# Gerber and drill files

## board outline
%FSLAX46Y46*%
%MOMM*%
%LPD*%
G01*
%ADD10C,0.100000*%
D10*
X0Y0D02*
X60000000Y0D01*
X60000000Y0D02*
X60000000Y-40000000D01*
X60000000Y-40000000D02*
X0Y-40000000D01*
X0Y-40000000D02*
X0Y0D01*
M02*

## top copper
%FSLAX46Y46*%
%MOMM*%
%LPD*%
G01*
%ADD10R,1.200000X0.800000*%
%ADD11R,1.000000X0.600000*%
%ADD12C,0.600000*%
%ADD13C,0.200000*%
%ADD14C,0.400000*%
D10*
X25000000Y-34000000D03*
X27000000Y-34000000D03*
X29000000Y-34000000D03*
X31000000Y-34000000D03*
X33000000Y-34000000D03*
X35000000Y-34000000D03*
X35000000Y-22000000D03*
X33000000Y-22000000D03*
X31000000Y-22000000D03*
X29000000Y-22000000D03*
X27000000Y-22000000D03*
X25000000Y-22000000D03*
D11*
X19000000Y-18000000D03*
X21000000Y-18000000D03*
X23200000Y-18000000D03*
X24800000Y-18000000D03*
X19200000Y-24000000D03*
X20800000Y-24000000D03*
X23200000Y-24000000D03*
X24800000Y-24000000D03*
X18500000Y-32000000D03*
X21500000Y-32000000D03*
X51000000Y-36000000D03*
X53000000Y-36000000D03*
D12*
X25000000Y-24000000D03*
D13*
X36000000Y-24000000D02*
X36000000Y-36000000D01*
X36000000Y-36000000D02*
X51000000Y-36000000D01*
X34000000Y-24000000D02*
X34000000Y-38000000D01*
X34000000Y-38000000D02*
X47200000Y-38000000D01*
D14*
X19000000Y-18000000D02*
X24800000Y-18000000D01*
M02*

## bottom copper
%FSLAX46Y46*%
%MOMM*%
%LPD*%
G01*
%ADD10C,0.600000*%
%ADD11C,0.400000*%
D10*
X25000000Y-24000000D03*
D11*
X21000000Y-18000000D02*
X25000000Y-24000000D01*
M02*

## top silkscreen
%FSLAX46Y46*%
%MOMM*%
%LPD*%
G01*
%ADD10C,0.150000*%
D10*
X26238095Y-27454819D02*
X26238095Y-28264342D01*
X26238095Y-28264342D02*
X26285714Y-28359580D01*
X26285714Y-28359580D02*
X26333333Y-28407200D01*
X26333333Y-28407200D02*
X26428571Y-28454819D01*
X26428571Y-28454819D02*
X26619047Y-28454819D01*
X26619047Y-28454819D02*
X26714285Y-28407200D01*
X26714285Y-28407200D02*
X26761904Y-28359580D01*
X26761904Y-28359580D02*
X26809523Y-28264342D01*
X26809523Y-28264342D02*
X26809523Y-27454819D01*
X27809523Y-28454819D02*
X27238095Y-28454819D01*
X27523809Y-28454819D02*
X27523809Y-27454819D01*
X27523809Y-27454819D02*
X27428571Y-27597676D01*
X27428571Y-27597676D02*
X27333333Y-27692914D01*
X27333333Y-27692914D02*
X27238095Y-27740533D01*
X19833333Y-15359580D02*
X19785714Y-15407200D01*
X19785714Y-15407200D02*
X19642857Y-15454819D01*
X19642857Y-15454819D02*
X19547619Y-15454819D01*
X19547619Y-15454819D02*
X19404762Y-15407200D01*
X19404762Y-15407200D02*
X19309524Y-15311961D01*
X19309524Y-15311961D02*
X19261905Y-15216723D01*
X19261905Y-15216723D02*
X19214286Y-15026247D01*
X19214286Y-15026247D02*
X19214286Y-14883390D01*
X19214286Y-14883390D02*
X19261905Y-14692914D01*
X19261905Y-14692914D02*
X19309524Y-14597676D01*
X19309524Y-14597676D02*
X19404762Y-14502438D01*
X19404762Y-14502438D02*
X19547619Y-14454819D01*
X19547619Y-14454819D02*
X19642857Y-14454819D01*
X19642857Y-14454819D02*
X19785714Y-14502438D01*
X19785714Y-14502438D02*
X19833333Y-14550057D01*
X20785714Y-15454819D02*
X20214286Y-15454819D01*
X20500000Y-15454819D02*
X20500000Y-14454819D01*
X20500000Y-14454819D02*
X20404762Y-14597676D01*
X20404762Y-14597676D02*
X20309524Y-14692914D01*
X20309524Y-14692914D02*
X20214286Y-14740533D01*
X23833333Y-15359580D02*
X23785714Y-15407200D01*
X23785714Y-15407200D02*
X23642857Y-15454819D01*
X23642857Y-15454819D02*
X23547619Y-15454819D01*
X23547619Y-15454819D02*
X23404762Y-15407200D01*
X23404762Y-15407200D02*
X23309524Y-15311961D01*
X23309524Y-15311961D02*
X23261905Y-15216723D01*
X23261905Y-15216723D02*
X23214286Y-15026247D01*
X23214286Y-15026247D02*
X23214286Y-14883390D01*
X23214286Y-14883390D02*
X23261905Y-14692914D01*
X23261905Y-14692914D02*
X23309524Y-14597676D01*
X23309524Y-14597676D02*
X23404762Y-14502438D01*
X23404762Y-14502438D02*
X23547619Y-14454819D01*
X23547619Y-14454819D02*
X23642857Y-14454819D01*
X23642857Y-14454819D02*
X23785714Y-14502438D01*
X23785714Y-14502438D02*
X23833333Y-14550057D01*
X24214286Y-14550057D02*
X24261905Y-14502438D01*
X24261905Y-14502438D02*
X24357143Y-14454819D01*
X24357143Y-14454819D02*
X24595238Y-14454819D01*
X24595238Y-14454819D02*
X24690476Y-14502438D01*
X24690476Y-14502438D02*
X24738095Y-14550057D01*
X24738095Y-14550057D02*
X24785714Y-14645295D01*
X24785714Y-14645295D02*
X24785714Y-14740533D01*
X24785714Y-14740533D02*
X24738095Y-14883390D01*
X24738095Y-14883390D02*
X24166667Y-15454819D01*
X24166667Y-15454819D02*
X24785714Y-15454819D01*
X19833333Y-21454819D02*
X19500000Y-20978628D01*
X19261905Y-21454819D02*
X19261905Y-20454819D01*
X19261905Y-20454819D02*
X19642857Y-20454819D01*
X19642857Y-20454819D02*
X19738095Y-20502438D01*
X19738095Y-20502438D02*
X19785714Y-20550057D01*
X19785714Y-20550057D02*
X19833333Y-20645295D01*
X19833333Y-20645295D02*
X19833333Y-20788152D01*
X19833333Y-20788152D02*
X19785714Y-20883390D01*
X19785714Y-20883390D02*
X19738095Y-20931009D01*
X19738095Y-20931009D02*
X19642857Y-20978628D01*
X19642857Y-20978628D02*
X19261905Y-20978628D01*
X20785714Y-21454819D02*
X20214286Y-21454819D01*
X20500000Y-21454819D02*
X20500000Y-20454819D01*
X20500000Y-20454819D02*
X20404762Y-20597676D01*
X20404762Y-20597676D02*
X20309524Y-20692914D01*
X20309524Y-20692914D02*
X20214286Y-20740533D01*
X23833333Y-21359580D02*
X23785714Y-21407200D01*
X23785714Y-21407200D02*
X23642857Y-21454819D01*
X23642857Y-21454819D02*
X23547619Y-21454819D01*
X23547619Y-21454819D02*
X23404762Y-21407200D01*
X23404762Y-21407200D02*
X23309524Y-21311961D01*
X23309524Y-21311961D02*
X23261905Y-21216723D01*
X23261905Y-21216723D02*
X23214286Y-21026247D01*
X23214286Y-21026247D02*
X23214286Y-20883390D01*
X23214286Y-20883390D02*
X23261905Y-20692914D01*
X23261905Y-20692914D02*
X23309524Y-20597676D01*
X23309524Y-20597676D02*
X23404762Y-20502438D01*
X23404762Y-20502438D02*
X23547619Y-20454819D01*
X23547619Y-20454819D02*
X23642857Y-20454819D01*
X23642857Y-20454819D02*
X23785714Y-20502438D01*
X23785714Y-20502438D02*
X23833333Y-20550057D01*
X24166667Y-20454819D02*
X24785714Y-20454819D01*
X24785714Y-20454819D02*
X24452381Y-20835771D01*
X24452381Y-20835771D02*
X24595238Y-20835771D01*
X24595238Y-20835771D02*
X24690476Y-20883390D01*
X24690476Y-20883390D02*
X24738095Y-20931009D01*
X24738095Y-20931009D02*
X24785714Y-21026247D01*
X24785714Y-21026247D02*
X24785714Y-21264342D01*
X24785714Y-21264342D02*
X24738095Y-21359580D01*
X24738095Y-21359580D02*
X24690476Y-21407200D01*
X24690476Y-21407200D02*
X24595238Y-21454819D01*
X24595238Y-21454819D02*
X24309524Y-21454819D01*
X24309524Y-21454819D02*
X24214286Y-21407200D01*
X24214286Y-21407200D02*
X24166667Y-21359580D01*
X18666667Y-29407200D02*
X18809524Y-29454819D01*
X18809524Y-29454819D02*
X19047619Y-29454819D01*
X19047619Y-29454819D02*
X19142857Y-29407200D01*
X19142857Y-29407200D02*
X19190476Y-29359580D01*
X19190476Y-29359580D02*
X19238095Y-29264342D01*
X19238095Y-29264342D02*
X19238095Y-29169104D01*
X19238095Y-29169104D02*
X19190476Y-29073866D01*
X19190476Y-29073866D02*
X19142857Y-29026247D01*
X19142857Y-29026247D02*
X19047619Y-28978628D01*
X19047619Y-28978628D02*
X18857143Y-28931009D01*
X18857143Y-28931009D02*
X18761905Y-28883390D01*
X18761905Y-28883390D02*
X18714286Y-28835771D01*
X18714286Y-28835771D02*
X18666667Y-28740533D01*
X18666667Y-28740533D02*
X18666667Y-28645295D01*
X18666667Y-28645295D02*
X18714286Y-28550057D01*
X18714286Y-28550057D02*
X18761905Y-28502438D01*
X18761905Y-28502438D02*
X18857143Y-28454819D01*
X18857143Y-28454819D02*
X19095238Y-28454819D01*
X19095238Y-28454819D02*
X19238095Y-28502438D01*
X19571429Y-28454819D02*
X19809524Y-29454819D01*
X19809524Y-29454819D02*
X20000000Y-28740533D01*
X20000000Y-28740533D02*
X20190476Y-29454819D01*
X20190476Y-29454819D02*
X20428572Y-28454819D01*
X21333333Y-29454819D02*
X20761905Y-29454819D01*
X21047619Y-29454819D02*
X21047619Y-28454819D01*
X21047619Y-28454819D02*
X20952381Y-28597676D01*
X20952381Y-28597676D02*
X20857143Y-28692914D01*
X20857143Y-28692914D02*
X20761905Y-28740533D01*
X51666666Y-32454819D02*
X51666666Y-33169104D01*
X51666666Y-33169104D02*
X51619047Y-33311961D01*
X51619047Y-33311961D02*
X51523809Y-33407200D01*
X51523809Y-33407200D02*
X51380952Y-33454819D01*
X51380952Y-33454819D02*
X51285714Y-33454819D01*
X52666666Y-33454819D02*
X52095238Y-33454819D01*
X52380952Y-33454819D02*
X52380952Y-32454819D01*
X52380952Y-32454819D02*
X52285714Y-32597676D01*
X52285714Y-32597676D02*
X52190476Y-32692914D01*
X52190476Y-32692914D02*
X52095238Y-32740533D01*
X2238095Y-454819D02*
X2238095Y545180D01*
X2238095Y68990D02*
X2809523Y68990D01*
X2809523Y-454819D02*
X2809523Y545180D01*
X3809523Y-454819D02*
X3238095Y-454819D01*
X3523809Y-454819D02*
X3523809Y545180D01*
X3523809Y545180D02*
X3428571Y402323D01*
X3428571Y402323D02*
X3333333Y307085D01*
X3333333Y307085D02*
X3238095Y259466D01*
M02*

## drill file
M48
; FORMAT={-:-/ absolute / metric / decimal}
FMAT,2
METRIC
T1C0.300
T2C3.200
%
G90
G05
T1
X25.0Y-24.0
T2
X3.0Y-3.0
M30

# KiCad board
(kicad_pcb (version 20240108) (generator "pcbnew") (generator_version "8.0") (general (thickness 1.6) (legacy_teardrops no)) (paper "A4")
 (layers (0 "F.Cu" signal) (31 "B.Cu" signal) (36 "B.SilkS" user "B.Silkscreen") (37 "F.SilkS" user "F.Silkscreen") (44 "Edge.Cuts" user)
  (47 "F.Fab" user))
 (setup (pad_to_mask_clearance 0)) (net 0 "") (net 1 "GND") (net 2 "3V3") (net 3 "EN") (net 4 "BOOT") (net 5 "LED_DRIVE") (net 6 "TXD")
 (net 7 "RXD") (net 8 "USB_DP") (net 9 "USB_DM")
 (gr_line (start 0 0) (end 60 0) (stroke (width 0.1) (type default)) (layer "Edge.Cuts"))
 (gr_line (start 60 0) (end 60 40) (stroke (width 0.1) (type default)) (layer "Edge.Cuts"))
 (gr_line (start 60 40) (end 0 40) (stroke (width 0.1) (type default)) (layer "Edge.Cuts"))
 (gr_line (start 0 40) (end 0 0) (stroke (width 0.1) (type default)) (layer "Edge.Cuts"))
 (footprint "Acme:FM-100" (layer "F.Cu") (at 30 28 90)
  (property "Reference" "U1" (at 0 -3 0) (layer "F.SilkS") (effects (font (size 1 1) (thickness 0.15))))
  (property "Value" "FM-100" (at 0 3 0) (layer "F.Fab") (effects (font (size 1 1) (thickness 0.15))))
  (pad "1" smd rect (at -6.0 -5.0 0) (size 1.2 0.8) (layers "F.Cu" "F.Paste" "F.Mask") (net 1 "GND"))
  (pad "2" smd rect (at -6.0 -3.0 0) (size 1.2 0.8) (layers "F.Cu" "F.Paste" "F.Mask") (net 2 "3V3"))
  (pad "3" smd rect (at -6.0 -1.0 0) (size 1.2 0.8) (layers "F.Cu" "F.Paste" "F.Mask") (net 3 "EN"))
  (pad "4" smd rect (at -6.0 1.0 0) (size 1.2 0.8) (layers "F.Cu" "F.Paste" "F.Mask") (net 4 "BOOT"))
  (pad "5" smd rect (at -6.0 3.0 0) (size 1.2 0.8) (layers "F.Cu" "F.Paste" "F.Mask") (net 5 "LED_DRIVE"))
  (pad "6" smd rect (at -6.0 5.0 0) (size 1.2 0.8) (layers "F.Cu" "F.Paste" "F.Mask") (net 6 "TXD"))
  (pad "7" smd rect (at 6.0 5.0 0) (size 1.2 0.8) (layers "F.Cu" "F.Paste" "F.Mask") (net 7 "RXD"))
  (pad "8" smd rect (at 6.0 3.0 0) (size 1.2 0.8) (layers "F.Cu" "F.Paste" "F.Mask") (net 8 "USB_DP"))
  (pad "9" smd rect (at 6.0 1.0 0) (size 1.2 0.8) (layers "F.Cu" "F.Paste" "F.Mask") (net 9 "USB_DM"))
  (pad "10" smd rect (at 6.0 -1.0 0) (size 1.2 0.8) (layers "F.Cu" "F.Paste" "F.Mask"))
  (pad "11" smd rect (at 6.0 -3.0 0) (size 1.2 0.8) (layers "F.Cu" "F.Paste" "F.Mask"))
  (pad "12" smd rect (at 6.0 -5.0 0) (size 1.2 0.8) (layers "F.Cu" "F.Paste" "F.Mask") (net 1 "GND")))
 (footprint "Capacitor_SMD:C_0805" (layer "F.Cu") (at 20 18 0)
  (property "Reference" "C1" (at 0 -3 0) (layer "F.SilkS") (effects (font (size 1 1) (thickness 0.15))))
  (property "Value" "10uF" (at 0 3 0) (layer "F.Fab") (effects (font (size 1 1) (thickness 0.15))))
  (pad "1" smd rect (at -1 0 0) (size 1.0 0.6) (layers "F.Cu" "F.Paste" "F.Mask") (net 2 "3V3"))
  (pad "2" smd rect (at 1 0 0) (size 1.0 0.6) (layers "F.Cu" "F.Paste" "F.Mask") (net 1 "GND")))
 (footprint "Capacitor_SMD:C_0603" (layer "F.Cu") (at 24 18 0)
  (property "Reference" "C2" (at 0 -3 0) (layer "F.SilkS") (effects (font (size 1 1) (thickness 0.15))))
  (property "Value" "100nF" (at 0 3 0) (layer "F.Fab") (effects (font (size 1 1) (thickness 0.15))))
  (pad "1" smd rect (at -0.8 0 0) (size 1.0 0.6) (layers "F.Cu" "F.Paste" "F.Mask") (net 2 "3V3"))
  (pad "2" smd rect (at 0.8 0 0) (size 1.0 0.6) (layers "F.Cu" "F.Paste" "F.Mask") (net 1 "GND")))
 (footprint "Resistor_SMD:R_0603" (layer "F.Cu") (at 20 24 0)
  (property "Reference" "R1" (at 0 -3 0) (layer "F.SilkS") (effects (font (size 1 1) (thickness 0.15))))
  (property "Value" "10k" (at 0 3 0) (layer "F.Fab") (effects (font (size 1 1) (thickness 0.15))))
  (pad "1" smd rect (at -0.8 0 0) (size 1.0 0.6) (layers "F.Cu" "F.Paste" "F.Mask") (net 2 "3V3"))
  (pad "2" smd rect (at 0.8 0 0) (size 1.0 0.6) (layers "F.Cu" "F.Paste" "F.Mask") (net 3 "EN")))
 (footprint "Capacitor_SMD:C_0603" (layer "F.Cu") (at 24 24 0)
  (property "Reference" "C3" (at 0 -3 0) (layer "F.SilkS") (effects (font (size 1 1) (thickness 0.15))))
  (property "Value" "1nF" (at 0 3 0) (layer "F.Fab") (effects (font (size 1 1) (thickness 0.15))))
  (pad "1" smd rect (at -0.8 0 0) (size 1.0 0.6) (layers "F.Cu" "F.Paste" "F.Mask") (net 3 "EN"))
  (pad "2" smd rect (at 0.8 0 0) (size 1.0 0.6) (layers "F.Cu" "F.Paste" "F.Mask") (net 1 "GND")))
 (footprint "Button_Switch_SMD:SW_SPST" (layer "F.Cu") (at 20 32 0)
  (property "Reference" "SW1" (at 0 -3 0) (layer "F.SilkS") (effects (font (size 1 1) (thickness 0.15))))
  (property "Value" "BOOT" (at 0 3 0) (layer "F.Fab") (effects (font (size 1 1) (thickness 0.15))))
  (pad "1" smd rect (at -1.5 0 0) (size 1.0 0.6) (layers "F.Cu" "F.Paste" "F.Mask") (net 4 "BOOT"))
  (pad "2" smd rect (at 1.5 0 0) (size 1.0 0.6) (layers "F.Cu" "F.Paste" "F.Mask") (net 1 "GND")))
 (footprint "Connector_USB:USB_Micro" (layer "F.Cu") (at 52 36 0)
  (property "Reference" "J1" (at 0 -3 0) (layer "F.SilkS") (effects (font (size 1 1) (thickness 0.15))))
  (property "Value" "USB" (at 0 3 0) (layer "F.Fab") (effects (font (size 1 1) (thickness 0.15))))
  (pad "1" smd rect (at -1 0 0) (size 1.0 0.6) (layers "F.Cu" "F.Paste" "F.Mask") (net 8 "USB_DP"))
  (pad "2" smd rect (at 1 0 0) (size 1.0 0.6) (layers "F.Cu" "F.Paste" "F.Mask") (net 9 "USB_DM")))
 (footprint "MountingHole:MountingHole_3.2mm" (layer "F.Cu") (at 3 3)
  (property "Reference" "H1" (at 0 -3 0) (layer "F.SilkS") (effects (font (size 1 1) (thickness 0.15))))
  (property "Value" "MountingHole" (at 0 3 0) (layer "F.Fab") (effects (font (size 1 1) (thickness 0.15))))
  (pad "" np_thru_hole circle (at 0 0) (size 3.2 3.2) (drill 3.2) (layers "*.Cu" "*.Mask")))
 (segment (start 36.0 24.0) (end 36.0 36.0) (width 0.2) (layer "F.Cu") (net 8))
 (segment (start 36.0 36.0) (end 51.0 36.0) (width 0.2) (layer "F.Cu") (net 8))
 (segment (start 34.0 24.0) (end 34.0 38.0) (width 0.2) (layer "F.Cu") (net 9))
 (segment (start 34.0 38.0) (end 47.2 38.0) (width 0.2) (layer "F.Cu") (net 9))
 (segment (start 19.0 18.0) (end 24.8 18.0) (width 0.4) (layer "F.Cu") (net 2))
 (segment (start 21.0 18.0) (end 25.0 24.0) (width 0.4) (layer "B.Cu") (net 1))
 (via (at 25.0 24.0) (size 0.6) (drill 0.3) (layers "F.Cu" "B.Cu") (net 1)))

